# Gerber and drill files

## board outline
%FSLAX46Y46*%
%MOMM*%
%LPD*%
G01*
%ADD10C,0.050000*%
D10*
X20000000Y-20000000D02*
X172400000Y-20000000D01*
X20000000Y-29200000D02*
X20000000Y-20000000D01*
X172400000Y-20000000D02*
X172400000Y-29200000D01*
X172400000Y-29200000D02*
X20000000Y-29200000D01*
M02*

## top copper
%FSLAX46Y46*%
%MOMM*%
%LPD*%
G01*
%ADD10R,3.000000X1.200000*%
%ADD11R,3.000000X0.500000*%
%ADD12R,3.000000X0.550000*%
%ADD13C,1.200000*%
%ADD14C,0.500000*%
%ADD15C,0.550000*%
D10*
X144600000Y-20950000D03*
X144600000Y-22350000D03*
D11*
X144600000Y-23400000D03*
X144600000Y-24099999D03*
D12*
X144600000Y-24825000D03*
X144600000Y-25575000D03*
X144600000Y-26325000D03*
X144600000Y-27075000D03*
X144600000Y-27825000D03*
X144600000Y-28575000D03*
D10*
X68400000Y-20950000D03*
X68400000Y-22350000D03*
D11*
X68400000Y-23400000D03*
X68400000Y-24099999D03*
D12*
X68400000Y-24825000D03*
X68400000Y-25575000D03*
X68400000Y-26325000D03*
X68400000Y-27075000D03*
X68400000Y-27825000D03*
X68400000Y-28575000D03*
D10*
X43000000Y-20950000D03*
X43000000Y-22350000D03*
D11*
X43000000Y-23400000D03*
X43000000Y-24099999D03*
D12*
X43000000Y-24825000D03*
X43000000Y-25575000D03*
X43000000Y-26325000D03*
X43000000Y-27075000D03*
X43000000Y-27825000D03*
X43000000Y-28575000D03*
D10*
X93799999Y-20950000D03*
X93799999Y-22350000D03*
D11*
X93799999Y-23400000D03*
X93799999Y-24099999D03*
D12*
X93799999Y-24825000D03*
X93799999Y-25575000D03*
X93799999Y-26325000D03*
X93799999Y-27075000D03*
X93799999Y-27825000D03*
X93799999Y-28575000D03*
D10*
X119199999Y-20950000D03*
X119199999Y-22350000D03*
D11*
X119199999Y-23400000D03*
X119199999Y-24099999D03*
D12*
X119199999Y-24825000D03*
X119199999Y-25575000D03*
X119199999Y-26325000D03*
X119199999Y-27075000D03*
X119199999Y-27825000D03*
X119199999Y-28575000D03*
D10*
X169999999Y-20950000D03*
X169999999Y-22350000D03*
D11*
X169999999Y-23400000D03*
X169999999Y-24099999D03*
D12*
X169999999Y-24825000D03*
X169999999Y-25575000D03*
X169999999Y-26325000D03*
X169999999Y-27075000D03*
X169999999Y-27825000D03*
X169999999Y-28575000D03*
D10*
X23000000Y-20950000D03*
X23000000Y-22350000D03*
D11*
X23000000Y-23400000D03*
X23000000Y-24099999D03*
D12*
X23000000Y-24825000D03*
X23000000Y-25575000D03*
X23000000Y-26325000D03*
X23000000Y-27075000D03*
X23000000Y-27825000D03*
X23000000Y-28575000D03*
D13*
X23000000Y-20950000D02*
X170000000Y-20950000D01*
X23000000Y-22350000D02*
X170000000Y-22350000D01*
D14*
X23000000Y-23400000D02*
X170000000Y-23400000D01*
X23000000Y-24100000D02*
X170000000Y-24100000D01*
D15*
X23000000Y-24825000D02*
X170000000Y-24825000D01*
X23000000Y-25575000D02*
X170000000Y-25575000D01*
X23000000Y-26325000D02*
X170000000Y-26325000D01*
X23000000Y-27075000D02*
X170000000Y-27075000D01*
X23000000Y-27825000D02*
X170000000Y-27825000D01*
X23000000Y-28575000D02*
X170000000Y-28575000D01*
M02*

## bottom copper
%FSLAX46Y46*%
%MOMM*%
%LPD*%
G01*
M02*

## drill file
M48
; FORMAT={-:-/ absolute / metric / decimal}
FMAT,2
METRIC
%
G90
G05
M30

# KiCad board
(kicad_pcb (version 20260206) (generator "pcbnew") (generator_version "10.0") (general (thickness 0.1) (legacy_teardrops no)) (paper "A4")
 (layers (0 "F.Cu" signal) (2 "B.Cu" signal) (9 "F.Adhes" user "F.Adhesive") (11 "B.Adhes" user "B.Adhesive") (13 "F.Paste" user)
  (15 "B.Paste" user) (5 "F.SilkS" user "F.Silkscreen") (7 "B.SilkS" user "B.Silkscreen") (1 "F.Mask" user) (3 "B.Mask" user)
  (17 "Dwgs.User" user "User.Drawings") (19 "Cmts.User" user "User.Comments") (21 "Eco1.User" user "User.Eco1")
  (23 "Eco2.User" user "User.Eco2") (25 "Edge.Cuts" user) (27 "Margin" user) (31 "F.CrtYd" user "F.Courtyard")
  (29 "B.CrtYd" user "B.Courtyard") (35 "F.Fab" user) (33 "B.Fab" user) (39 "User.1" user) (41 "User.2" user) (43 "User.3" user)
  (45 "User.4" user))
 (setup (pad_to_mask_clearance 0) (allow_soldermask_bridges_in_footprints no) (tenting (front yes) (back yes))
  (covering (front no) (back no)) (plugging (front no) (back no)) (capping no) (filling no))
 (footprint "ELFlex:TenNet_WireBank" (layer "F.Cu") (at 144.6 20)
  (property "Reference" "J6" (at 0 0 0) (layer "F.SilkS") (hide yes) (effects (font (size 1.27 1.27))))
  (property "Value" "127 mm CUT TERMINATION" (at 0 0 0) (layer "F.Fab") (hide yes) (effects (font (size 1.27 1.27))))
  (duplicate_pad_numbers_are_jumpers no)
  (pad "1" smd rect (at 0 0.95) (size 3 1.2) (layers "F.Cu" "F.Mask") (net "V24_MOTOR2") (solder_mask_margin -0.05)
   (thermal_bridge_angle 45))
  (pad "2" smd rect (at 0 2.35) (size 3 1.2) (layers "F.Cu" "F.Mask") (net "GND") (solder_mask_margin -0.05) (thermal_bridge_angle 45))
  (pad "3" smd rect (at 0 3.4) (size 3 0.5) (layers "F.Cu" "F.Mask") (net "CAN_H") (solder_mask_margin -0.05) (thermal_bridge_angle 45))
  (pad "4" smd rect (at 0 4.099999) (size 3 0.5) (layers "F.Cu" "F.Mask") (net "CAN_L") (solder_mask_margin -0.05) (thermal_bridge_angle 45))
  (pad "5" smd rect (at 0 4.825) (size 3 0.55) (layers "F.Cu" "F.Mask") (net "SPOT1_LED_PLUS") (solder_mask_margin -0.05)
   (thermal_bridge_angle 45))
  (pad "6" smd rect (at 0 5.575) (size 3 0.55) (layers "F.Cu" "F.Mask") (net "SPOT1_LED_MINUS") (solder_mask_margin -0.05)
   (thermal_bridge_angle 45))
  (pad "7" smd rect (at 0 6.325) (size 3 0.55) (layers "F.Cu" "F.Mask") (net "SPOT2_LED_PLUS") (solder_mask_margin -0.05)
   (thermal_bridge_angle 45))
  (pad "8" smd rect (at 0 7.075) (size 3 0.55) (layers "F.Cu" "F.Mask") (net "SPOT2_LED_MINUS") (solder_mask_margin -0.05)
   (thermal_bridge_angle 45))
  (pad "9" smd rect (at 0 7.825) (size 3 0.55) (layers "F.Cu" "F.Mask") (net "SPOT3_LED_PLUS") (solder_mask_margin -0.05)
   (thermal_bridge_angle 45))
  (pad "10" smd rect (at 0 8.575) (size 3 0.55) (layers "F.Cu" "F.Mask") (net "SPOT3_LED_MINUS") (solder_mask_margin -0.05)
   (thermal_bridge_angle 45)))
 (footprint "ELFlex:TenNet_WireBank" (layer "F.Cu") (at 68.4 20)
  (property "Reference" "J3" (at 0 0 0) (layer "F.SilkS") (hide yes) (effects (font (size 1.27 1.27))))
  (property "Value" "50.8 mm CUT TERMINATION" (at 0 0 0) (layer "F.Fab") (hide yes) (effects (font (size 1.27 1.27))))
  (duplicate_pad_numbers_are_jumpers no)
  (pad "1" smd rect (at 0 0.95) (size 3 1.2) (layers "F.Cu" "F.Mask") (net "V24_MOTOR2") (solder_mask_margin -0.05)
   (thermal_bridge_angle 45))
  (pad "2" smd rect (at 0 2.35) (size 3 1.2) (layers "F.Cu" "F.Mask") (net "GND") (solder_mask_margin -0.05) (thermal_bridge_angle 45))
  (pad "3" smd rect (at 0 3.4) (size 3 0.5) (layers "F.Cu" "F.Mask") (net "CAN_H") (solder_mask_margin -0.05) (thermal_bridge_angle 45))
  (pad "4" smd rect (at 0 4.099999) (size 3 0.5) (layers "F.Cu" "F.Mask") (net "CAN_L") (solder_mask_margin -0.05) (thermal_bridge_angle 45))
  (pad "5" smd rect (at 0 4.825) (size 3 0.55) (layers "F.Cu" "F.Mask") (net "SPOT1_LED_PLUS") (solder_mask_margin -0.05)
   (thermal_bridge_angle 45))
  (pad "6" smd rect (at 0 5.575) (size 3 0.55) (layers "F.Cu" "F.Mask") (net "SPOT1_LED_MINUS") (solder_mask_margin -0.05)
   (thermal_bridge_angle 45))
  (pad "7" smd rect (at 0 6.325) (size 3 0.55) (layers "F.Cu" "F.Mask") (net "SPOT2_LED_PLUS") (solder_mask_margin -0.05)
   (thermal_bridge_angle 45))
  (pad "8" smd rect (at 0 7.075) (size 3 0.55) (layers "F.Cu" "F.Mask") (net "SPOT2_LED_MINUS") (solder_mask_margin -0.05)
   (thermal_bridge_angle 45))
  (pad "9" smd rect (at 0 7.825) (size 3 0.55) (layers "F.Cu" "F.Mask") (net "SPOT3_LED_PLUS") (solder_mask_margin -0.05)
   (thermal_bridge_angle 45))
  (pad "10" smd rect (at 0 8.575) (size 3 0.55) (layers "F.Cu" "F.Mask") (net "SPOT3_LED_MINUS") (solder_mask_margin -0.05)
   (thermal_bridge_angle 45)))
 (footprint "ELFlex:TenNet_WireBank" (layer "F.Cu") (at 43 20)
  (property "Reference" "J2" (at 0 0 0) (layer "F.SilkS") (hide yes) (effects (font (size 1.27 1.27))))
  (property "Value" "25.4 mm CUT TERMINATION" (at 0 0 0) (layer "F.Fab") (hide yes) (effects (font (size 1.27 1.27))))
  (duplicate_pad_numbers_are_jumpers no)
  (pad "1" smd rect (at 0 0.95) (size 3 1.2) (layers "F.Cu" "F.Mask") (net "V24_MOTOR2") (solder_mask_margin -0.05)
   (thermal_bridge_angle 45))
  (pad "2" smd rect (at 0 2.35) (size 3 1.2) (layers "F.Cu" "F.Mask") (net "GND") (solder_mask_margin -0.05) (thermal_bridge_angle 45))
  (pad "3" smd rect (at 0 3.4) (size 3 0.5) (layers "F.Cu" "F.Mask") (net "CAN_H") (solder_mask_margin -0.05) (thermal_bridge_angle 45))
  (pad "4" smd rect (at 0 4.099999) (size 3 0.5) (layers "F.Cu" "F.Mask") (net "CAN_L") (solder_mask_margin -0.05) (thermal_bridge_angle 45))
  (pad "5" smd rect (at 0 4.825) (size 3 0.55) (layers "F.Cu" "F.Mask") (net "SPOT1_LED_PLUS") (solder_mask_margin -0.05)
   (thermal_bridge_angle 45))
  (pad "6" smd rect (at 0 5.575) (size 3 0.55) (layers "F.Cu" "F.Mask") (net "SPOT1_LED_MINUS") (solder_mask_margin -0.05)
   (thermal_bridge_angle 45))
  (pad "7" smd rect (at 0 6.325) (size 3 0.55) (layers "F.Cu" "F.Mask") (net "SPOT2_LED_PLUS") (solder_mask_margin -0.05)
   (thermal_bridge_angle 45))
  (pad "8" smd rect (at 0 7.075) (size 3 0.55) (layers "F.Cu" "F.Mask") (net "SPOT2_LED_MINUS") (solder_mask_margin -0.05)
   (thermal_bridge_angle 45))
  (pad "9" smd rect (at 0 7.825) (size 3 0.55) (layers "F.Cu" "F.Mask") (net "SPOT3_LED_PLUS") (solder_mask_margin -0.05)
   (thermal_bridge_angle 45))
  (pad "10" smd rect (at 0 8.575) (size 3 0.55) (layers "F.Cu" "F.Mask") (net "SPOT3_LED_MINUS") (solder_mask_margin -0.05)
   (thermal_bridge_angle 45)))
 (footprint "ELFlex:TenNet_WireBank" (layer "F.Cu") (at 93.799999 20)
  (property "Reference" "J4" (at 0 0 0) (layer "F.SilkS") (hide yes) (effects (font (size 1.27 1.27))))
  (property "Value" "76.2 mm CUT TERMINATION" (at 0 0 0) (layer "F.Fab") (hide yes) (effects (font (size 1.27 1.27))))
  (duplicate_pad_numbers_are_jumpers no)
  (pad "1" smd rect (at 0 0.95) (size 3 1.2) (layers "F.Cu" "F.Mask") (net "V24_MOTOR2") (solder_mask_margin -0.05)
   (thermal_bridge_angle 45))
  (pad "2" smd rect (at 0 2.35) (size 3 1.2) (layers "F.Cu" "F.Mask") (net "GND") (solder_mask_margin -0.05) (thermal_bridge_angle 45))
  (pad "3" smd rect (at 0 3.4) (size 3 0.5) (layers "F.Cu" "F.Mask") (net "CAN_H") (solder_mask_margin -0.05) (thermal_bridge_angle 45))
  (pad "4" smd rect (at 0 4.099999) (size 3 0.5) (layers "F.Cu" "F.Mask") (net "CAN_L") (solder_mask_margin -0.05) (thermal_bridge_angle 45))
  (pad "5" smd rect (at 0 4.825) (size 3 0.55) (layers "F.Cu" "F.Mask") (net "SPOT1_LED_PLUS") (solder_mask_margin -0.05)
   (thermal_bridge_angle 45))
  (pad "6" smd rect (at 0 5.575) (size 3 0.55) (layers "F.Cu" "F.Mask") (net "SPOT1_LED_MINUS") (solder_mask_margin -0.05)
   (thermal_bridge_angle 45))
  (pad "7" smd rect (at 0 6.325) (size 3 0.55) (layers "F.Cu" "F.Mask") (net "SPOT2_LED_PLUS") (solder_mask_margin -0.05)
   (thermal_bridge_angle 45))
  (pad "8" smd rect (at 0 7.075) (size 3 0.55) (layers "F.Cu" "F.Mask") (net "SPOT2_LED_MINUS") (solder_mask_margin -0.05)
   (thermal_bridge_angle 45))
  (pad "9" smd rect (at 0 7.825) (size 3 0.55) (layers "F.Cu" "F.Mask") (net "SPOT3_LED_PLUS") (solder_mask_margin -0.05)
   (thermal_bridge_angle 45))
  (pad "10" smd rect (at 0 8.575) (size 3 0.55) (layers "F.Cu" "F.Mask") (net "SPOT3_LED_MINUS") (solder_mask_margin -0.05)
   (thermal_bridge_angle 45)))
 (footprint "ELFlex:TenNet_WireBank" (layer "F.Cu") (at 119.199999 20)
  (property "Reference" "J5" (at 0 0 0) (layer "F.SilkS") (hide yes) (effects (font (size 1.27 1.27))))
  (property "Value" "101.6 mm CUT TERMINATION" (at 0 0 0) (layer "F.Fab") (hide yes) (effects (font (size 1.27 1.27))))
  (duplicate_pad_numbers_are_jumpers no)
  (pad "1" smd rect (at 0 0.95) (size 3 1.2) (layers "F.Cu" "F.Mask") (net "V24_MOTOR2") (solder_mask_margin -0.05)
   (thermal_bridge_angle 45))
  (pad "2" smd rect (at 0 2.35) (size 3 1.2) (layers "F.Cu" "F.Mask") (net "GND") (solder_mask_margin -0.05) (thermal_bridge_angle 45))
  (pad "3" smd rect (at 0 3.4) (size 3 0.5) (layers "F.Cu" "F.Mask") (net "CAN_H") (solder_mask_margin -0.05) (thermal_bridge_angle 45))
  (pad "4" smd rect (at 0 4.099999) (size 3 0.5) (layers "F.Cu" "F.Mask") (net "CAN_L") (solder_mask_margin -0.05) (thermal_bridge_angle 45))
  (pad "5" smd rect (at 0 4.825) (size 3 0.55) (layers "F.Cu" "F.Mask") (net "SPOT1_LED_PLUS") (solder_mask_margin -0.05)
   (thermal_bridge_angle 45))
  (pad "6" smd rect (at 0 5.575) (size 3 0.55) (layers "F.Cu" "F.Mask") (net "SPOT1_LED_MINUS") (solder_mask_margin -0.05)
   (thermal_bridge_angle 45))
  (pad "7" smd rect (at 0 6.325) (size 3 0.55) (layers "F.Cu" "F.Mask") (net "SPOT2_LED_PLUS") (solder_mask_margin -0.05)
   (thermal_bridge_angle 45))
  (pad "8" smd rect (at 0 7.075) (size 3 0.55) (layers "F.Cu" "F.Mask") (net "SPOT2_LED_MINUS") (solder_mask_margin -0.05)
   (thermal_bridge_angle 45))
  (pad "9" smd rect (at 0 7.825) (size 3 0.55) (layers "F.Cu" "F.Mask") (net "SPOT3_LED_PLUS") (solder_mask_margin -0.05)
   (thermal_bridge_angle 45))
  (pad "10" smd rect (at 0 8.575) (size 3 0.55) (layers "F.Cu" "F.Mask") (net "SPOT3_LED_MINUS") (solder_mask_margin -0.05)
   (thermal_bridge_angle 45)))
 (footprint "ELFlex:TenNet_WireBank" (layer "F.Cu") (at 169.999999 20)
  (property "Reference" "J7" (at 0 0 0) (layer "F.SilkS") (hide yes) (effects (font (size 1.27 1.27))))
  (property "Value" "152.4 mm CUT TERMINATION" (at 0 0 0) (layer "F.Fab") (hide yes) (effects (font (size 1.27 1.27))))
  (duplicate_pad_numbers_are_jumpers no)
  (pad "1" smd rect (at 0 0.95) (size 3 1.2) (layers "F.Cu" "F.Mask") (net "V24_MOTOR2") (solder_mask_margin -0.05)
   (thermal_bridge_angle 45))
  (pad "2" smd rect (at 0 2.35) (size 3 1.2) (layers "F.Cu" "F.Mask") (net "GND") (solder_mask_margin -0.05) (thermal_bridge_angle 45))
  (pad "3" smd rect (at 0 3.4) (size 3 0.5) (layers "F.Cu" "F.Mask") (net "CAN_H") (solder_mask_margin -0.05) (thermal_bridge_angle 45))
  (pad "4" smd rect (at 0 4.099999) (size 3 0.5) (layers "F.Cu" "F.Mask") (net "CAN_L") (solder_mask_margin -0.05) (thermal_bridge_angle 45))
  (pad "5" smd rect (at 0 4.825) (size 3 0.55) (layers "F.Cu" "F.Mask") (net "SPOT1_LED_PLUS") (solder_mask_margin -0.05)
   (thermal_bridge_angle 45))
  (pad "6" smd rect (at 0 5.575) (size 3 0.55) (layers "F.Cu" "F.Mask") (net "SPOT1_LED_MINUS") (solder_mask_margin -0.05)
   (thermal_bridge_angle 45))
  (pad "7" smd rect (at 0 6.325) (size 3 0.55) (layers "F.Cu" "F.Mask") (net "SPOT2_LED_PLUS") (solder_mask_margin -0.05)
   (thermal_bridge_angle 45))
  (pad "8" smd rect (at 0 7.075) (size 3 0.55) (layers "F.Cu" "F.Mask") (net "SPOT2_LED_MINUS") (solder_mask_margin -0.05)
   (thermal_bridge_angle 45))
  (pad "9" smd rect (at 0 7.825) (size 3 0.55) (layers "F.Cu" "F.Mask") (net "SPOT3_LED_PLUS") (solder_mask_margin -0.05)
   (thermal_bridge_angle 45))
  (pad "10" smd rect (at 0 8.575) (size 3 0.55) (layers "F.Cu" "F.Mask") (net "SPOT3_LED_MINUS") (solder_mask_margin -0.05)
   (thermal_bridge_angle 45)))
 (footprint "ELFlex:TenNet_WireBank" (layer "F.Cu") (at 23 20)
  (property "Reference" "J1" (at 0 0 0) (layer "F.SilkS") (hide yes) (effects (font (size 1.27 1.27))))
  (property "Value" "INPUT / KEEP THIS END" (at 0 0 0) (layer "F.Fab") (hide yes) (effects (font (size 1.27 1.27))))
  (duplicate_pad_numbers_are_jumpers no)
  (pad "1" smd rect (at 0 0.95) (size 3 1.2) (layers "F.Cu" "F.Mask") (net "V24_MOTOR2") (solder_mask_margin -0.05)
   (thermal_bridge_angle 45))
  (pad "2" smd rect (at 0 2.35) (size 3 1.2) (layers "F.Cu" "F.Mask") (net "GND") (solder_mask_margin -0.05) (thermal_bridge_angle 45))
  (pad "3" smd rect (at 0 3.4) (size 3 0.5) (layers "F.Cu" "F.Mask") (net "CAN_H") (solder_mask_margin -0.05) (thermal_bridge_angle 45))
  (pad "4" smd rect (at 0 4.099999) (size 3 0.5) (layers "F.Cu" "F.Mask") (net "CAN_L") (solder_mask_margin -0.05) (thermal_bridge_angle 45))
  (pad "5" smd rect (at 0 4.825) (size 3 0.55) (layers "F.Cu" "F.Mask") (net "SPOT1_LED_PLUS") (solder_mask_margin -0.05)
   (thermal_bridge_angle 45))
  (pad "6" smd rect (at 0 5.575) (size 3 0.55) (layers "F.Cu" "F.Mask") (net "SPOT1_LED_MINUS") (solder_mask_margin -0.05)
   (thermal_bridge_angle 45))
  (pad "7" smd rect (at 0 6.325) (size 3 0.55) (layers "F.Cu" "F.Mask") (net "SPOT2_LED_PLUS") (solder_mask_margin -0.05)
   (thermal_bridge_angle 45))
  (pad "8" smd rect (at 0 7.075) (size 3 0.55) (layers "F.Cu" "F.Mask") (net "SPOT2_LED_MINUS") (solder_mask_margin -0.05)
   (thermal_bridge_angle 45))
  (pad "9" smd rect (at 0 7.825) (size 3 0.55) (layers "F.Cu" "F.Mask") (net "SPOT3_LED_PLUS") (solder_mask_margin -0.05)
   (thermal_bridge_angle 45))
  (pad "10" smd rect (at 0 8.575) (size 3 0.55) (layers "F.Cu" "F.Mask") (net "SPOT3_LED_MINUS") (solder_mask_margin -0.05)
   (thermal_bridge_angle 45)))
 (gr_line (start 20 20) (end 172.4 20) (stroke (width 0.05) (type default)) (layer "Edge.Cuts"))
 (gr_line (start 20 29.2) (end 20 20) (stroke (width 0.05) (type default)) (layer "Edge.Cuts"))
 (gr_line (start 172.4 20) (end 172.4 29.2) (stroke (width 0.05) (type default)) (layer "Edge.Cuts"))
 (gr_line (start 172.4 29.2) (end 20 29.2) (stroke (width 0.05) (type default)) (layer "Edge.Cuts"))
 (segment (start 23 20.95) (end 170 20.95) (width 1.2) (layer "F.Cu") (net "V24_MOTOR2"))
 (segment (start 23 22.35) (end 170 22.35) (width 1.2) (layer "F.Cu") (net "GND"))
 (segment (start 23 23.4) (end 170 23.4) (width 0.5) (layer "F.Cu") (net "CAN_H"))
 (segment (start 23 24.1) (end 170 24.1) (width 0.5) (layer "F.Cu") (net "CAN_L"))
 (segment (start 23 24.825) (end 170 24.825) (width 0.55) (layer "F.Cu") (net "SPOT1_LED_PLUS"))
 (segment (start 23 25.575) (end 170 25.575) (width 0.55) (layer "F.Cu") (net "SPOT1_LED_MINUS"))
 (segment (start 23 26.325) (end 170 26.325) (width 0.55) (layer "F.Cu") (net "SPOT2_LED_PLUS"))
 (segment (start 23 27.075) (end 170 27.075) (width 0.55) (layer "F.Cu") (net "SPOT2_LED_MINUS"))
 (segment (start 23 27.825) (end 170 27.825) (width 0.55) (layer "F.Cu") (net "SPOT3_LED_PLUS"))
 (segment (start 23 28.575) (end 170 28.575) (width 0.55) (layer "F.Cu") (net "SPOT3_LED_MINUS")))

